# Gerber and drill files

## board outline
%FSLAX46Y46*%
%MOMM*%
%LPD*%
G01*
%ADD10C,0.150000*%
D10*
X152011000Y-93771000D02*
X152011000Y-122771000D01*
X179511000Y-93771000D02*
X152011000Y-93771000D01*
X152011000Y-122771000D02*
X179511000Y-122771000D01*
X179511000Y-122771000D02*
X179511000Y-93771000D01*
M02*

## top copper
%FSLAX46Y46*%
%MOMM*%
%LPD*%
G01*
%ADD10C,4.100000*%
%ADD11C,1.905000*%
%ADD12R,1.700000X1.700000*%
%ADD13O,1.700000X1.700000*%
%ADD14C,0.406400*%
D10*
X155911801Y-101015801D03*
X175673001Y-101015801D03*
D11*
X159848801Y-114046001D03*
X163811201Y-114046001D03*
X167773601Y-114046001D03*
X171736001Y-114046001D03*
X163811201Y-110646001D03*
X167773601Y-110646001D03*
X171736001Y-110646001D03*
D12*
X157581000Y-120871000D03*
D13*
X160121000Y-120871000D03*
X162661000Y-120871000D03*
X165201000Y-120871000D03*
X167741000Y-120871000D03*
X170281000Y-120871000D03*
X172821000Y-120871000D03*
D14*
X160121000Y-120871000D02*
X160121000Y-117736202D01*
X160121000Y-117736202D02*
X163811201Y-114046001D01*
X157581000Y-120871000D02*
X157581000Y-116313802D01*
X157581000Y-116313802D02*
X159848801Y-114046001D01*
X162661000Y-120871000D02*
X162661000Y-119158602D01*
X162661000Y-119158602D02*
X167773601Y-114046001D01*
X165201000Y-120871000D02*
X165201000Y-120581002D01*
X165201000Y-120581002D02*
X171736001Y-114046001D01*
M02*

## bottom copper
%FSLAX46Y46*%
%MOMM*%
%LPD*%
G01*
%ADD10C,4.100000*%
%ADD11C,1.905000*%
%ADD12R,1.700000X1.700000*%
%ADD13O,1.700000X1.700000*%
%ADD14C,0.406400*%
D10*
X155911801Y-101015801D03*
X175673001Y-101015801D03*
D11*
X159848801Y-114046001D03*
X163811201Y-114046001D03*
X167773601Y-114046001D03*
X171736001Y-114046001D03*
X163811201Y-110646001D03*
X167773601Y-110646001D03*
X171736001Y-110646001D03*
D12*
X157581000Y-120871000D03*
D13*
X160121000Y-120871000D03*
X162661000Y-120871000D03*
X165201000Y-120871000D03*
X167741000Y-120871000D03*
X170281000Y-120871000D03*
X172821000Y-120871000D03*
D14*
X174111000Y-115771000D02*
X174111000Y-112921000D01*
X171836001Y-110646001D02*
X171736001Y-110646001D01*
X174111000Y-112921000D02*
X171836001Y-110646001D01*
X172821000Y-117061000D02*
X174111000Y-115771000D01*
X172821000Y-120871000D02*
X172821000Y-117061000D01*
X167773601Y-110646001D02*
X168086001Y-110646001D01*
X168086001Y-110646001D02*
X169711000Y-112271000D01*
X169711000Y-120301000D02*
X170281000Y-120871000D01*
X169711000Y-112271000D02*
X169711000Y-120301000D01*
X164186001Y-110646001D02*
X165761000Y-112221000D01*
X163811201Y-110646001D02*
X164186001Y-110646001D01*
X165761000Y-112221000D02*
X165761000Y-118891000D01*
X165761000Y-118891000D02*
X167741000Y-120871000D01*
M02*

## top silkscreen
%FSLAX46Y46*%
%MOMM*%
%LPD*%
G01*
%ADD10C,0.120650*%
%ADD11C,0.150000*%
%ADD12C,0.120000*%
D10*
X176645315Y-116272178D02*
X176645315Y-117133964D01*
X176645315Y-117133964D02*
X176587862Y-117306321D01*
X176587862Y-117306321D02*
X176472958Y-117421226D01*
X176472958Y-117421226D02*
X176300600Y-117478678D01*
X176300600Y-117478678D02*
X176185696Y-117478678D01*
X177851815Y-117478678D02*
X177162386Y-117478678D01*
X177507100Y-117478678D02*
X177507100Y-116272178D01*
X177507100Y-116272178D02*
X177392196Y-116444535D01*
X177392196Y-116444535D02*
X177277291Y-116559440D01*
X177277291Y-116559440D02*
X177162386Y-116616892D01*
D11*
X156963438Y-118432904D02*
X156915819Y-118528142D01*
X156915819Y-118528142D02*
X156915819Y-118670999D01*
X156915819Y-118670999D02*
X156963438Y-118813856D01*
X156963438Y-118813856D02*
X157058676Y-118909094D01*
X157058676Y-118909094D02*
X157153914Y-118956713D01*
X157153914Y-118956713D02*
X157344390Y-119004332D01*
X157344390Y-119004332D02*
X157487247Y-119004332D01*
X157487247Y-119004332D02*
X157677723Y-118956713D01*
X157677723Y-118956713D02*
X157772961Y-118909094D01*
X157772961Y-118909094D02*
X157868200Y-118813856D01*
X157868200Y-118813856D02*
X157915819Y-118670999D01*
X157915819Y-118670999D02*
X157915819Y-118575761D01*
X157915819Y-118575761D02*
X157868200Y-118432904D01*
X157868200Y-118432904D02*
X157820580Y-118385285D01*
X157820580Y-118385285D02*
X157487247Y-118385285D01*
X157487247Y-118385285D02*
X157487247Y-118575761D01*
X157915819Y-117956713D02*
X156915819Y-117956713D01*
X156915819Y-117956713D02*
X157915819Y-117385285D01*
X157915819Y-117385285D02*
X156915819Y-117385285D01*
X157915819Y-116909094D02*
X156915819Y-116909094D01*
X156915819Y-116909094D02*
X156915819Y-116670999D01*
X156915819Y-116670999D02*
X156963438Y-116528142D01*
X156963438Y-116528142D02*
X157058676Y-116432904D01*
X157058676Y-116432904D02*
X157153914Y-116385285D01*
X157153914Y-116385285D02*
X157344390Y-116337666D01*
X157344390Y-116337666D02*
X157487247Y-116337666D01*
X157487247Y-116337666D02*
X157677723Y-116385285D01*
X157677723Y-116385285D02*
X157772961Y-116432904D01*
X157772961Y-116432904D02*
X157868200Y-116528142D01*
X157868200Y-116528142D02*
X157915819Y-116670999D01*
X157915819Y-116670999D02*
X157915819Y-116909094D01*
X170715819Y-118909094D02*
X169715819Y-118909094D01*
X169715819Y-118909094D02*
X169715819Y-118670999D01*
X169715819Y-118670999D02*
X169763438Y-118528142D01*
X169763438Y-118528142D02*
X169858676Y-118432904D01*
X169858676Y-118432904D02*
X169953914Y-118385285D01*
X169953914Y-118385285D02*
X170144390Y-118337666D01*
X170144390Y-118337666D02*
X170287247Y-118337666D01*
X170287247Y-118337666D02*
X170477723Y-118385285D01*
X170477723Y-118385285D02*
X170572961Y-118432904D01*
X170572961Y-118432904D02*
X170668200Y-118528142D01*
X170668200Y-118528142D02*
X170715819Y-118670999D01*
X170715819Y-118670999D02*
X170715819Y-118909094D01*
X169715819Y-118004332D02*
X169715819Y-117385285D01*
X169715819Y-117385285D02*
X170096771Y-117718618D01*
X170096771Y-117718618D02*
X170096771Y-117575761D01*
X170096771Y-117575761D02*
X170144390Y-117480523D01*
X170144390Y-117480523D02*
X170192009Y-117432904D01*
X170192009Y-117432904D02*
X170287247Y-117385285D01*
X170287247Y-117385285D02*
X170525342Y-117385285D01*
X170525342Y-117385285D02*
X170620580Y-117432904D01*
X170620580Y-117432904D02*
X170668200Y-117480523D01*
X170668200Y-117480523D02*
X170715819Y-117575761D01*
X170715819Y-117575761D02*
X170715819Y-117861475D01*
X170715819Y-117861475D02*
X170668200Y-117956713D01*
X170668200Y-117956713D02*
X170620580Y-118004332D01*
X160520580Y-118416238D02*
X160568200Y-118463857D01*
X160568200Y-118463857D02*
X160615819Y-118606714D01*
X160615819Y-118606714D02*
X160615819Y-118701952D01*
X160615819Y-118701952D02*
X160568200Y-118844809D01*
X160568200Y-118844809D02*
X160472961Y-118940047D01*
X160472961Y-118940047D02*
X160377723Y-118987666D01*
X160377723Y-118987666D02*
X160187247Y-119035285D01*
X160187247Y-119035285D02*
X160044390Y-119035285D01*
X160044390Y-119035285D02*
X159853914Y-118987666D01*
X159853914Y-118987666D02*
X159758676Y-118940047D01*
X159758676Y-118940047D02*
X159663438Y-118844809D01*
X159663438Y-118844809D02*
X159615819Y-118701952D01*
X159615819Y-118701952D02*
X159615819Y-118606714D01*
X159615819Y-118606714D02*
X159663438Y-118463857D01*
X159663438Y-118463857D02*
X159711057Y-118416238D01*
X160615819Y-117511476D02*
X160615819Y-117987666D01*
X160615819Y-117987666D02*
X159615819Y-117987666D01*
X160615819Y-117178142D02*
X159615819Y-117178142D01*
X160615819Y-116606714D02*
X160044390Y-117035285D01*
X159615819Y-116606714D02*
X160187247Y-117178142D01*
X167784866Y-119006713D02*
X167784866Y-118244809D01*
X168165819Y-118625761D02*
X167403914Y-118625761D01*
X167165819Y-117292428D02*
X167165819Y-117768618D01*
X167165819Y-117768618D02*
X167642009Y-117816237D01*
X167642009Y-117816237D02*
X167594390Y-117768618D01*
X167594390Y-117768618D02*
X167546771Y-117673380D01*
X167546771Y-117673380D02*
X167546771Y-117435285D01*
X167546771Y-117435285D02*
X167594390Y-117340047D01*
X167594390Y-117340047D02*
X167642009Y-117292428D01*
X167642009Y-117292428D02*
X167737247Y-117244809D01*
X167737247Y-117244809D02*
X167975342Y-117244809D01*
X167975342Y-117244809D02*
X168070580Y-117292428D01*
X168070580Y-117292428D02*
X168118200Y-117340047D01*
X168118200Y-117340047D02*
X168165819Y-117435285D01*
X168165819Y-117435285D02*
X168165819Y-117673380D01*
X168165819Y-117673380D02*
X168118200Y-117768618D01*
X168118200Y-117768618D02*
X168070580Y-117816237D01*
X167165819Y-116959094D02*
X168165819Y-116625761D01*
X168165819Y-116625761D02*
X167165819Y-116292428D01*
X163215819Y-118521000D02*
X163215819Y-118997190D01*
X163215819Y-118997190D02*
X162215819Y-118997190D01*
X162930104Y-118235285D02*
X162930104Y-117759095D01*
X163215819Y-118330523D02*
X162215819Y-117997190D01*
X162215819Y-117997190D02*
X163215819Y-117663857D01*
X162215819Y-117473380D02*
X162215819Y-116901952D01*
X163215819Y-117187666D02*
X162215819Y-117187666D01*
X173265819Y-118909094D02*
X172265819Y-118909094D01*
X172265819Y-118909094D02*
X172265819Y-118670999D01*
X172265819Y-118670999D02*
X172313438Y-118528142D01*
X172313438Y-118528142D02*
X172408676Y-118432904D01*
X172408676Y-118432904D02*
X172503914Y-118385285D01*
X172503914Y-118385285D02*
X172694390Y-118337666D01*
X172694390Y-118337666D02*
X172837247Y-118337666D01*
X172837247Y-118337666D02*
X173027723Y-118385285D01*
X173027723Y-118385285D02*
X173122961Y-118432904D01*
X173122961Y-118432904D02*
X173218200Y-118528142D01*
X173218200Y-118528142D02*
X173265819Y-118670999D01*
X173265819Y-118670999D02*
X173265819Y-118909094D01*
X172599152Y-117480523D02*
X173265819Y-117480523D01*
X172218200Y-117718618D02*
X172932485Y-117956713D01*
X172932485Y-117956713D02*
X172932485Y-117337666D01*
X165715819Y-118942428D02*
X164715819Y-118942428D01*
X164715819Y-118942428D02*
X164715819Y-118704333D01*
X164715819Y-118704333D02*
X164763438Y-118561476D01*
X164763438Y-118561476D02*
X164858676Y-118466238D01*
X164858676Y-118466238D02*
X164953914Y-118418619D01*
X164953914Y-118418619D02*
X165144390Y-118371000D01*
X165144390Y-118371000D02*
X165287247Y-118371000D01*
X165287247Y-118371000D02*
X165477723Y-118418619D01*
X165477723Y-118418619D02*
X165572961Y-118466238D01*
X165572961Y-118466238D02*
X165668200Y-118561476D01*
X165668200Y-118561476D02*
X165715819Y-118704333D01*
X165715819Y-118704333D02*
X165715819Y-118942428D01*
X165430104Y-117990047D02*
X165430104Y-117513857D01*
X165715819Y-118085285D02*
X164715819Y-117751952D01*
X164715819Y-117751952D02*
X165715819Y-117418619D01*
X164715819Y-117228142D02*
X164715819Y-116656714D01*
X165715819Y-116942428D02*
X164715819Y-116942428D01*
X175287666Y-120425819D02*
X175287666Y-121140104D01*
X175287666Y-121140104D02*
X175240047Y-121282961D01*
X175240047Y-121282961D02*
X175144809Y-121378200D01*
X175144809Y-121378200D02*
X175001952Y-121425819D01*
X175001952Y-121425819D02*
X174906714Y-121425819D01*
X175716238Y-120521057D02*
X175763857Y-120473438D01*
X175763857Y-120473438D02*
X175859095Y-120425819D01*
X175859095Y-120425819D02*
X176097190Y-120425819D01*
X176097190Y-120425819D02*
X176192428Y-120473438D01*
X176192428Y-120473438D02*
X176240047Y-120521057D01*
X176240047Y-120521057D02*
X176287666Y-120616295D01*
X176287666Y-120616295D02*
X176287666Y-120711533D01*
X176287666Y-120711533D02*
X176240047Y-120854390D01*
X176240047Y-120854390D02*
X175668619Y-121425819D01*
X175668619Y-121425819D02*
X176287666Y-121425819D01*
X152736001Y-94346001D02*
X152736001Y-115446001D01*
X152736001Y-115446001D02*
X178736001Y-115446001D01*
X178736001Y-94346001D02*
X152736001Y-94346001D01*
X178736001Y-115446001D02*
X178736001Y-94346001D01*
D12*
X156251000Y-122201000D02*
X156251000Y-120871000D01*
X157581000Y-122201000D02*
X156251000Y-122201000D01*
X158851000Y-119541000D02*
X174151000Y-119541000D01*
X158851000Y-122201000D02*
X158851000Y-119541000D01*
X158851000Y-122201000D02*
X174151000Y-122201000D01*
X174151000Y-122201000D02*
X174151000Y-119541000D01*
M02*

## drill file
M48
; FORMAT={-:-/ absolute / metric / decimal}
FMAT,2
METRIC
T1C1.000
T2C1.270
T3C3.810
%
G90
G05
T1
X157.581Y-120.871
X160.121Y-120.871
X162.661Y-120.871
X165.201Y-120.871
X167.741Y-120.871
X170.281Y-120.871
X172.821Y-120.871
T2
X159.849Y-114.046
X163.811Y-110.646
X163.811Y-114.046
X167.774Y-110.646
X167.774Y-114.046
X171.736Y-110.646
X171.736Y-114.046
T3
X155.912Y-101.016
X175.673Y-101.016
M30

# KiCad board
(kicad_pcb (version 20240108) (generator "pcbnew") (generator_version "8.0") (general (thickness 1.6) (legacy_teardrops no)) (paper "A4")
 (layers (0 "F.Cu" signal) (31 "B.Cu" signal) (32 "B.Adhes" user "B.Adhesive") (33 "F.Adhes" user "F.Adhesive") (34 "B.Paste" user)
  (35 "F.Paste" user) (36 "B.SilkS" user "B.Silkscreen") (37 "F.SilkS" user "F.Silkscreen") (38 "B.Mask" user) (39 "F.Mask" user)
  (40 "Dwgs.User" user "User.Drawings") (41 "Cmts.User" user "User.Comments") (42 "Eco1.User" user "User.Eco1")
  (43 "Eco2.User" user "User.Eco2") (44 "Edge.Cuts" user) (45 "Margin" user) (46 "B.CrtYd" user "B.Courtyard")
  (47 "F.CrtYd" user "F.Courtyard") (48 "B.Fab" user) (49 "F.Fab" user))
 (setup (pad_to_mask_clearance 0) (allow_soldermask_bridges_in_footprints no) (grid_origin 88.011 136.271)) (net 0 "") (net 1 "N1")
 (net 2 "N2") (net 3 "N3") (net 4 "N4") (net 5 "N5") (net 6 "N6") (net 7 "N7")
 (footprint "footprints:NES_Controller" (layer "F.Cu") (at 171.736001 114.046001)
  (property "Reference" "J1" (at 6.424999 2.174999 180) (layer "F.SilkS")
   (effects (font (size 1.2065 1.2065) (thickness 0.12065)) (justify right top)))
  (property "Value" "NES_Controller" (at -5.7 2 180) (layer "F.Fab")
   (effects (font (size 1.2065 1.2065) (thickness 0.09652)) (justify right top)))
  (fp_line (start -19 -19.7) (end -19 1.4) (stroke (width 0.15) (type solid)) (layer "F.SilkS"))
  (fp_line (start -19 1.4) (end 7 1.4) (stroke (width 0.15) (type solid)) (layer "F.SilkS"))
  (fp_line (start 7 -19.7) (end -19 -19.7) (stroke (width 0.15) (type solid)) (layer "F.SilkS"))
  (fp_line (start 7 1.4) (end 7 -19.7) (stroke (width 0.15) (type solid)) (layer "F.SilkS"))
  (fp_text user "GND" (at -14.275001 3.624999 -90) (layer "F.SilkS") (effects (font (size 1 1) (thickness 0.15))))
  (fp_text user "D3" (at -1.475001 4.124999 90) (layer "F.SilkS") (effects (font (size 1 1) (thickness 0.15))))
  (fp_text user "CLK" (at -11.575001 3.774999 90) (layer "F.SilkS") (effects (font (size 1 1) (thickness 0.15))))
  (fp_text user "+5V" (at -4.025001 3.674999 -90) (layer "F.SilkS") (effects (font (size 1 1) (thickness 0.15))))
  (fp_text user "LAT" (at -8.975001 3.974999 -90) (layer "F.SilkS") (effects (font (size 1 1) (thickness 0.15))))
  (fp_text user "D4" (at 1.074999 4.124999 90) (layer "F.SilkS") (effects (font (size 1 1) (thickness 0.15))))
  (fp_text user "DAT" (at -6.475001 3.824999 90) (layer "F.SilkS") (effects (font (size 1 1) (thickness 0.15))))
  (pad "" np_thru_hole circle (at -15.8242 -13.0302) (size 4.1 4.1) (drill 3.81) (layers "F&B.Cu" "*.Mask"))
  (pad "" np_thru_hole circle (at 3.937 -13.0302) (size 4.1 4.1) (drill 3.81) (layers "F&B.Cu" "*.Mask"))
  (pad "1" thru_hole circle (at -11.8872 0) (size 1.905 1.905) (drill 1.27) (layers "*.Cu" "*.Mask") (remove_unused_layers no) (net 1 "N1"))
  (pad "2" thru_hole circle (at -7.9248 0) (size 1.905 1.905) (drill 1.27) (layers "*.Cu" "*.Mask") (remove_unused_layers no) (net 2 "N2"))
  (pad "3" thru_hole circle (at -3.9624 0) (size 1.905 1.905) (drill 1.27) (layers "*.Cu" "*.Mask") (remove_unused_layers no) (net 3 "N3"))
  (pad "4" thru_hole circle (at 0 0) (size 1.905 1.905) (drill 1.27) (layers "*.Cu" "*.Mask") (remove_unused_layers no) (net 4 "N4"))
  (pad "5" thru_hole circle (at -7.9248 -3.4) (size 1.905 1.905) (drill 1.27) (layers "*.Cu" "*.Mask") (remove_unused_layers no)
   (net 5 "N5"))
  (pad "6" thru_hole circle (at -3.9624 -3.4) (size 1.905 1.905) (drill 1.27) (layers "*.Cu" "*.Mask") (remove_unused_layers no)
   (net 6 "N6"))
  (pad "7" thru_hole circle (at 0 -3.4) (size 1.905 1.905) (drill 1.27) (layers "*.Cu" "*.Mask") (remove_unused_layers no) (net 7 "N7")))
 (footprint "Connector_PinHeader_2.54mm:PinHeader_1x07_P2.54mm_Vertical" (layer "F.Cu") (at 157.581 120.871 90)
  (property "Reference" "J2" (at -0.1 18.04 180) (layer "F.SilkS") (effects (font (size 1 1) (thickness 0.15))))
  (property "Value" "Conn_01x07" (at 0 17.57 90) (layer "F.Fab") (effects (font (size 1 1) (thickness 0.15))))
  (fp_line (start -1.33 -1.33) (end 0 -1.33) (stroke (width 0.12) (type solid)) (layer "F.SilkS"))
  (fp_line (start -1.33 0) (end -1.33 -1.33) (stroke (width 0.12) (type solid)) (layer "F.SilkS"))
  (fp_line (start 1.33 1.27) (end 1.33 16.57) (stroke (width 0.12) (type solid)) (layer "F.SilkS"))
  (fp_line (start -1.33 1.27) (end 1.33 1.27) (stroke (width 0.12) (type solid)) (layer "F.SilkS"))
  (fp_line (start -1.33 1.27) (end -1.33 16.57) (stroke (width 0.12) (type solid)) (layer "F.SilkS"))
  (fp_line (start -1.33 16.57) (end 1.33 16.57) (stroke (width 0.12) (type solid)) (layer "F.SilkS"))
  (pad "1" thru_hole rect (at 0 0 90) (size 1.7 1.7) (drill 1) (layers "*.Cu" "*.Mask") (remove_unused_layers no) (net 1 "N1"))
  (pad "2" thru_hole oval (at 0 2.54 90) (size 1.7 1.7) (drill 1) (layers "*.Cu" "*.Mask") (remove_unused_layers no) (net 2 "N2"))
  (pad "3" thru_hole oval (at 0 5.08 90) (size 1.7 1.7) (drill 1) (layers "*.Cu" "*.Mask") (remove_unused_layers no) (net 3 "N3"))
  (pad "4" thru_hole oval (at 0 7.62 90) (size 1.7 1.7) (drill 1) (layers "*.Cu" "*.Mask") (remove_unused_layers no) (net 4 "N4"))
  (pad "5" thru_hole oval (at 0 10.16 90) (size 1.7 1.7) (drill 1) (layers "*.Cu" "*.Mask") (remove_unused_layers no) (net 5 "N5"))
  (pad "6" thru_hole oval (at 0 12.7 90) (size 1.7 1.7) (drill 1) (layers "*.Cu" "*.Mask") (remove_unused_layers no) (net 6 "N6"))
  (pad "7" thru_hole oval (at 0 15.24 90) (size 1.7 1.7) (drill 1) (layers "*.Cu" "*.Mask") (remove_unused_layers no) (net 7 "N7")))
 (gr_line (start 152.011 93.771) (end 152.011 122.771) (stroke (width 0.15) (type solid)) (layer "Edge.Cuts"))
 (gr_line (start 179.511 93.771) (end 152.011 93.771) (stroke (width 0.15) (type solid)) (layer "Edge.Cuts"))
 (gr_line (start 152.011 122.771) (end 179.511 122.771) (stroke (width 0.15) (type solid)) (layer "Edge.Cuts"))
 (gr_line (start 179.511 122.771) (end 179.511 93.771) (stroke (width 0.15) (type solid)) (layer "Edge.Cuts"))
 (segment (start 160.121 120.871) (end 160.121 117.736202) (width 0.4064) (layer "F.Cu") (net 2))
 (segment (start 160.121 117.736202) (end 163.811201 114.046001) (width 0.4064) (layer "F.Cu") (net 2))
 (segment (start 157.581 120.871) (end 157.581 116.313802) (width 0.4064) (layer "F.Cu") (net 1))
 (segment (start 157.581 116.313802) (end 159.848801 114.046001) (width 0.4064) (layer "F.Cu") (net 1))
 (segment (start 162.661 120.871) (end 162.661 119.158602) (width 0.4064) (layer "F.Cu") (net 3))
 (segment (start 162.661 119.158602) (end 167.773601 114.046001) (width 0.4064) (layer "F.Cu") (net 3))
 (segment (start 165.201 120.871) (end 165.201 120.581002) (width 0.4064) (layer "F.Cu") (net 4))
 (segment (start 165.201 120.581002) (end 171.736001 114.046001) (width 0.4064) (layer "F.Cu") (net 4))
 (segment (start 174.111 115.771) (end 174.111 112.921) (width 0.4064) (layer "B.Cu") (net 7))
 (segment (start 171.836001 110.646001) (end 171.736001 110.646001) (width 0.4064) (layer "B.Cu") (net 7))
 (segment (start 174.111 112.921) (end 171.836001 110.646001) (width 0.4064) (layer "B.Cu") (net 7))
 (segment (start 172.821 117.061) (end 174.111 115.771) (width 0.4064) (layer "B.Cu") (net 7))
 (segment (start 172.821 120.871) (end 172.821 117.061) (width 0.4064) (layer "B.Cu") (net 7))
 (segment (start 167.773601 110.646001) (end 168.086001 110.646001) (width 0.4064) (layer "B.Cu") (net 6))
 (segment (start 168.086001 110.646001) (end 169.711 112.271) (width 0.4064) (layer "B.Cu") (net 6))
 (segment (start 169.711 120.301) (end 170.281 120.871) (width 0.4064) (layer "B.Cu") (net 6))
 (segment (start 169.711 112.271) (end 169.711 120.301) (width 0.4064) (layer "B.Cu") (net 6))
 (segment (start 164.186001 110.646001) (end 165.761 112.221) (width 0.4064) (layer "B.Cu") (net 5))
 (segment (start 163.811201 110.646001) (end 164.186001 110.646001) (width 0.4064) (layer "B.Cu") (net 5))
 (segment (start 165.761 112.221) (end 165.761 118.891) (width 0.4064) (layer "B.Cu") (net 5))
 (segment (start 165.761 118.891) (end 167.741 120.871) (width 0.4064) (layer "B.Cu") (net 5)))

